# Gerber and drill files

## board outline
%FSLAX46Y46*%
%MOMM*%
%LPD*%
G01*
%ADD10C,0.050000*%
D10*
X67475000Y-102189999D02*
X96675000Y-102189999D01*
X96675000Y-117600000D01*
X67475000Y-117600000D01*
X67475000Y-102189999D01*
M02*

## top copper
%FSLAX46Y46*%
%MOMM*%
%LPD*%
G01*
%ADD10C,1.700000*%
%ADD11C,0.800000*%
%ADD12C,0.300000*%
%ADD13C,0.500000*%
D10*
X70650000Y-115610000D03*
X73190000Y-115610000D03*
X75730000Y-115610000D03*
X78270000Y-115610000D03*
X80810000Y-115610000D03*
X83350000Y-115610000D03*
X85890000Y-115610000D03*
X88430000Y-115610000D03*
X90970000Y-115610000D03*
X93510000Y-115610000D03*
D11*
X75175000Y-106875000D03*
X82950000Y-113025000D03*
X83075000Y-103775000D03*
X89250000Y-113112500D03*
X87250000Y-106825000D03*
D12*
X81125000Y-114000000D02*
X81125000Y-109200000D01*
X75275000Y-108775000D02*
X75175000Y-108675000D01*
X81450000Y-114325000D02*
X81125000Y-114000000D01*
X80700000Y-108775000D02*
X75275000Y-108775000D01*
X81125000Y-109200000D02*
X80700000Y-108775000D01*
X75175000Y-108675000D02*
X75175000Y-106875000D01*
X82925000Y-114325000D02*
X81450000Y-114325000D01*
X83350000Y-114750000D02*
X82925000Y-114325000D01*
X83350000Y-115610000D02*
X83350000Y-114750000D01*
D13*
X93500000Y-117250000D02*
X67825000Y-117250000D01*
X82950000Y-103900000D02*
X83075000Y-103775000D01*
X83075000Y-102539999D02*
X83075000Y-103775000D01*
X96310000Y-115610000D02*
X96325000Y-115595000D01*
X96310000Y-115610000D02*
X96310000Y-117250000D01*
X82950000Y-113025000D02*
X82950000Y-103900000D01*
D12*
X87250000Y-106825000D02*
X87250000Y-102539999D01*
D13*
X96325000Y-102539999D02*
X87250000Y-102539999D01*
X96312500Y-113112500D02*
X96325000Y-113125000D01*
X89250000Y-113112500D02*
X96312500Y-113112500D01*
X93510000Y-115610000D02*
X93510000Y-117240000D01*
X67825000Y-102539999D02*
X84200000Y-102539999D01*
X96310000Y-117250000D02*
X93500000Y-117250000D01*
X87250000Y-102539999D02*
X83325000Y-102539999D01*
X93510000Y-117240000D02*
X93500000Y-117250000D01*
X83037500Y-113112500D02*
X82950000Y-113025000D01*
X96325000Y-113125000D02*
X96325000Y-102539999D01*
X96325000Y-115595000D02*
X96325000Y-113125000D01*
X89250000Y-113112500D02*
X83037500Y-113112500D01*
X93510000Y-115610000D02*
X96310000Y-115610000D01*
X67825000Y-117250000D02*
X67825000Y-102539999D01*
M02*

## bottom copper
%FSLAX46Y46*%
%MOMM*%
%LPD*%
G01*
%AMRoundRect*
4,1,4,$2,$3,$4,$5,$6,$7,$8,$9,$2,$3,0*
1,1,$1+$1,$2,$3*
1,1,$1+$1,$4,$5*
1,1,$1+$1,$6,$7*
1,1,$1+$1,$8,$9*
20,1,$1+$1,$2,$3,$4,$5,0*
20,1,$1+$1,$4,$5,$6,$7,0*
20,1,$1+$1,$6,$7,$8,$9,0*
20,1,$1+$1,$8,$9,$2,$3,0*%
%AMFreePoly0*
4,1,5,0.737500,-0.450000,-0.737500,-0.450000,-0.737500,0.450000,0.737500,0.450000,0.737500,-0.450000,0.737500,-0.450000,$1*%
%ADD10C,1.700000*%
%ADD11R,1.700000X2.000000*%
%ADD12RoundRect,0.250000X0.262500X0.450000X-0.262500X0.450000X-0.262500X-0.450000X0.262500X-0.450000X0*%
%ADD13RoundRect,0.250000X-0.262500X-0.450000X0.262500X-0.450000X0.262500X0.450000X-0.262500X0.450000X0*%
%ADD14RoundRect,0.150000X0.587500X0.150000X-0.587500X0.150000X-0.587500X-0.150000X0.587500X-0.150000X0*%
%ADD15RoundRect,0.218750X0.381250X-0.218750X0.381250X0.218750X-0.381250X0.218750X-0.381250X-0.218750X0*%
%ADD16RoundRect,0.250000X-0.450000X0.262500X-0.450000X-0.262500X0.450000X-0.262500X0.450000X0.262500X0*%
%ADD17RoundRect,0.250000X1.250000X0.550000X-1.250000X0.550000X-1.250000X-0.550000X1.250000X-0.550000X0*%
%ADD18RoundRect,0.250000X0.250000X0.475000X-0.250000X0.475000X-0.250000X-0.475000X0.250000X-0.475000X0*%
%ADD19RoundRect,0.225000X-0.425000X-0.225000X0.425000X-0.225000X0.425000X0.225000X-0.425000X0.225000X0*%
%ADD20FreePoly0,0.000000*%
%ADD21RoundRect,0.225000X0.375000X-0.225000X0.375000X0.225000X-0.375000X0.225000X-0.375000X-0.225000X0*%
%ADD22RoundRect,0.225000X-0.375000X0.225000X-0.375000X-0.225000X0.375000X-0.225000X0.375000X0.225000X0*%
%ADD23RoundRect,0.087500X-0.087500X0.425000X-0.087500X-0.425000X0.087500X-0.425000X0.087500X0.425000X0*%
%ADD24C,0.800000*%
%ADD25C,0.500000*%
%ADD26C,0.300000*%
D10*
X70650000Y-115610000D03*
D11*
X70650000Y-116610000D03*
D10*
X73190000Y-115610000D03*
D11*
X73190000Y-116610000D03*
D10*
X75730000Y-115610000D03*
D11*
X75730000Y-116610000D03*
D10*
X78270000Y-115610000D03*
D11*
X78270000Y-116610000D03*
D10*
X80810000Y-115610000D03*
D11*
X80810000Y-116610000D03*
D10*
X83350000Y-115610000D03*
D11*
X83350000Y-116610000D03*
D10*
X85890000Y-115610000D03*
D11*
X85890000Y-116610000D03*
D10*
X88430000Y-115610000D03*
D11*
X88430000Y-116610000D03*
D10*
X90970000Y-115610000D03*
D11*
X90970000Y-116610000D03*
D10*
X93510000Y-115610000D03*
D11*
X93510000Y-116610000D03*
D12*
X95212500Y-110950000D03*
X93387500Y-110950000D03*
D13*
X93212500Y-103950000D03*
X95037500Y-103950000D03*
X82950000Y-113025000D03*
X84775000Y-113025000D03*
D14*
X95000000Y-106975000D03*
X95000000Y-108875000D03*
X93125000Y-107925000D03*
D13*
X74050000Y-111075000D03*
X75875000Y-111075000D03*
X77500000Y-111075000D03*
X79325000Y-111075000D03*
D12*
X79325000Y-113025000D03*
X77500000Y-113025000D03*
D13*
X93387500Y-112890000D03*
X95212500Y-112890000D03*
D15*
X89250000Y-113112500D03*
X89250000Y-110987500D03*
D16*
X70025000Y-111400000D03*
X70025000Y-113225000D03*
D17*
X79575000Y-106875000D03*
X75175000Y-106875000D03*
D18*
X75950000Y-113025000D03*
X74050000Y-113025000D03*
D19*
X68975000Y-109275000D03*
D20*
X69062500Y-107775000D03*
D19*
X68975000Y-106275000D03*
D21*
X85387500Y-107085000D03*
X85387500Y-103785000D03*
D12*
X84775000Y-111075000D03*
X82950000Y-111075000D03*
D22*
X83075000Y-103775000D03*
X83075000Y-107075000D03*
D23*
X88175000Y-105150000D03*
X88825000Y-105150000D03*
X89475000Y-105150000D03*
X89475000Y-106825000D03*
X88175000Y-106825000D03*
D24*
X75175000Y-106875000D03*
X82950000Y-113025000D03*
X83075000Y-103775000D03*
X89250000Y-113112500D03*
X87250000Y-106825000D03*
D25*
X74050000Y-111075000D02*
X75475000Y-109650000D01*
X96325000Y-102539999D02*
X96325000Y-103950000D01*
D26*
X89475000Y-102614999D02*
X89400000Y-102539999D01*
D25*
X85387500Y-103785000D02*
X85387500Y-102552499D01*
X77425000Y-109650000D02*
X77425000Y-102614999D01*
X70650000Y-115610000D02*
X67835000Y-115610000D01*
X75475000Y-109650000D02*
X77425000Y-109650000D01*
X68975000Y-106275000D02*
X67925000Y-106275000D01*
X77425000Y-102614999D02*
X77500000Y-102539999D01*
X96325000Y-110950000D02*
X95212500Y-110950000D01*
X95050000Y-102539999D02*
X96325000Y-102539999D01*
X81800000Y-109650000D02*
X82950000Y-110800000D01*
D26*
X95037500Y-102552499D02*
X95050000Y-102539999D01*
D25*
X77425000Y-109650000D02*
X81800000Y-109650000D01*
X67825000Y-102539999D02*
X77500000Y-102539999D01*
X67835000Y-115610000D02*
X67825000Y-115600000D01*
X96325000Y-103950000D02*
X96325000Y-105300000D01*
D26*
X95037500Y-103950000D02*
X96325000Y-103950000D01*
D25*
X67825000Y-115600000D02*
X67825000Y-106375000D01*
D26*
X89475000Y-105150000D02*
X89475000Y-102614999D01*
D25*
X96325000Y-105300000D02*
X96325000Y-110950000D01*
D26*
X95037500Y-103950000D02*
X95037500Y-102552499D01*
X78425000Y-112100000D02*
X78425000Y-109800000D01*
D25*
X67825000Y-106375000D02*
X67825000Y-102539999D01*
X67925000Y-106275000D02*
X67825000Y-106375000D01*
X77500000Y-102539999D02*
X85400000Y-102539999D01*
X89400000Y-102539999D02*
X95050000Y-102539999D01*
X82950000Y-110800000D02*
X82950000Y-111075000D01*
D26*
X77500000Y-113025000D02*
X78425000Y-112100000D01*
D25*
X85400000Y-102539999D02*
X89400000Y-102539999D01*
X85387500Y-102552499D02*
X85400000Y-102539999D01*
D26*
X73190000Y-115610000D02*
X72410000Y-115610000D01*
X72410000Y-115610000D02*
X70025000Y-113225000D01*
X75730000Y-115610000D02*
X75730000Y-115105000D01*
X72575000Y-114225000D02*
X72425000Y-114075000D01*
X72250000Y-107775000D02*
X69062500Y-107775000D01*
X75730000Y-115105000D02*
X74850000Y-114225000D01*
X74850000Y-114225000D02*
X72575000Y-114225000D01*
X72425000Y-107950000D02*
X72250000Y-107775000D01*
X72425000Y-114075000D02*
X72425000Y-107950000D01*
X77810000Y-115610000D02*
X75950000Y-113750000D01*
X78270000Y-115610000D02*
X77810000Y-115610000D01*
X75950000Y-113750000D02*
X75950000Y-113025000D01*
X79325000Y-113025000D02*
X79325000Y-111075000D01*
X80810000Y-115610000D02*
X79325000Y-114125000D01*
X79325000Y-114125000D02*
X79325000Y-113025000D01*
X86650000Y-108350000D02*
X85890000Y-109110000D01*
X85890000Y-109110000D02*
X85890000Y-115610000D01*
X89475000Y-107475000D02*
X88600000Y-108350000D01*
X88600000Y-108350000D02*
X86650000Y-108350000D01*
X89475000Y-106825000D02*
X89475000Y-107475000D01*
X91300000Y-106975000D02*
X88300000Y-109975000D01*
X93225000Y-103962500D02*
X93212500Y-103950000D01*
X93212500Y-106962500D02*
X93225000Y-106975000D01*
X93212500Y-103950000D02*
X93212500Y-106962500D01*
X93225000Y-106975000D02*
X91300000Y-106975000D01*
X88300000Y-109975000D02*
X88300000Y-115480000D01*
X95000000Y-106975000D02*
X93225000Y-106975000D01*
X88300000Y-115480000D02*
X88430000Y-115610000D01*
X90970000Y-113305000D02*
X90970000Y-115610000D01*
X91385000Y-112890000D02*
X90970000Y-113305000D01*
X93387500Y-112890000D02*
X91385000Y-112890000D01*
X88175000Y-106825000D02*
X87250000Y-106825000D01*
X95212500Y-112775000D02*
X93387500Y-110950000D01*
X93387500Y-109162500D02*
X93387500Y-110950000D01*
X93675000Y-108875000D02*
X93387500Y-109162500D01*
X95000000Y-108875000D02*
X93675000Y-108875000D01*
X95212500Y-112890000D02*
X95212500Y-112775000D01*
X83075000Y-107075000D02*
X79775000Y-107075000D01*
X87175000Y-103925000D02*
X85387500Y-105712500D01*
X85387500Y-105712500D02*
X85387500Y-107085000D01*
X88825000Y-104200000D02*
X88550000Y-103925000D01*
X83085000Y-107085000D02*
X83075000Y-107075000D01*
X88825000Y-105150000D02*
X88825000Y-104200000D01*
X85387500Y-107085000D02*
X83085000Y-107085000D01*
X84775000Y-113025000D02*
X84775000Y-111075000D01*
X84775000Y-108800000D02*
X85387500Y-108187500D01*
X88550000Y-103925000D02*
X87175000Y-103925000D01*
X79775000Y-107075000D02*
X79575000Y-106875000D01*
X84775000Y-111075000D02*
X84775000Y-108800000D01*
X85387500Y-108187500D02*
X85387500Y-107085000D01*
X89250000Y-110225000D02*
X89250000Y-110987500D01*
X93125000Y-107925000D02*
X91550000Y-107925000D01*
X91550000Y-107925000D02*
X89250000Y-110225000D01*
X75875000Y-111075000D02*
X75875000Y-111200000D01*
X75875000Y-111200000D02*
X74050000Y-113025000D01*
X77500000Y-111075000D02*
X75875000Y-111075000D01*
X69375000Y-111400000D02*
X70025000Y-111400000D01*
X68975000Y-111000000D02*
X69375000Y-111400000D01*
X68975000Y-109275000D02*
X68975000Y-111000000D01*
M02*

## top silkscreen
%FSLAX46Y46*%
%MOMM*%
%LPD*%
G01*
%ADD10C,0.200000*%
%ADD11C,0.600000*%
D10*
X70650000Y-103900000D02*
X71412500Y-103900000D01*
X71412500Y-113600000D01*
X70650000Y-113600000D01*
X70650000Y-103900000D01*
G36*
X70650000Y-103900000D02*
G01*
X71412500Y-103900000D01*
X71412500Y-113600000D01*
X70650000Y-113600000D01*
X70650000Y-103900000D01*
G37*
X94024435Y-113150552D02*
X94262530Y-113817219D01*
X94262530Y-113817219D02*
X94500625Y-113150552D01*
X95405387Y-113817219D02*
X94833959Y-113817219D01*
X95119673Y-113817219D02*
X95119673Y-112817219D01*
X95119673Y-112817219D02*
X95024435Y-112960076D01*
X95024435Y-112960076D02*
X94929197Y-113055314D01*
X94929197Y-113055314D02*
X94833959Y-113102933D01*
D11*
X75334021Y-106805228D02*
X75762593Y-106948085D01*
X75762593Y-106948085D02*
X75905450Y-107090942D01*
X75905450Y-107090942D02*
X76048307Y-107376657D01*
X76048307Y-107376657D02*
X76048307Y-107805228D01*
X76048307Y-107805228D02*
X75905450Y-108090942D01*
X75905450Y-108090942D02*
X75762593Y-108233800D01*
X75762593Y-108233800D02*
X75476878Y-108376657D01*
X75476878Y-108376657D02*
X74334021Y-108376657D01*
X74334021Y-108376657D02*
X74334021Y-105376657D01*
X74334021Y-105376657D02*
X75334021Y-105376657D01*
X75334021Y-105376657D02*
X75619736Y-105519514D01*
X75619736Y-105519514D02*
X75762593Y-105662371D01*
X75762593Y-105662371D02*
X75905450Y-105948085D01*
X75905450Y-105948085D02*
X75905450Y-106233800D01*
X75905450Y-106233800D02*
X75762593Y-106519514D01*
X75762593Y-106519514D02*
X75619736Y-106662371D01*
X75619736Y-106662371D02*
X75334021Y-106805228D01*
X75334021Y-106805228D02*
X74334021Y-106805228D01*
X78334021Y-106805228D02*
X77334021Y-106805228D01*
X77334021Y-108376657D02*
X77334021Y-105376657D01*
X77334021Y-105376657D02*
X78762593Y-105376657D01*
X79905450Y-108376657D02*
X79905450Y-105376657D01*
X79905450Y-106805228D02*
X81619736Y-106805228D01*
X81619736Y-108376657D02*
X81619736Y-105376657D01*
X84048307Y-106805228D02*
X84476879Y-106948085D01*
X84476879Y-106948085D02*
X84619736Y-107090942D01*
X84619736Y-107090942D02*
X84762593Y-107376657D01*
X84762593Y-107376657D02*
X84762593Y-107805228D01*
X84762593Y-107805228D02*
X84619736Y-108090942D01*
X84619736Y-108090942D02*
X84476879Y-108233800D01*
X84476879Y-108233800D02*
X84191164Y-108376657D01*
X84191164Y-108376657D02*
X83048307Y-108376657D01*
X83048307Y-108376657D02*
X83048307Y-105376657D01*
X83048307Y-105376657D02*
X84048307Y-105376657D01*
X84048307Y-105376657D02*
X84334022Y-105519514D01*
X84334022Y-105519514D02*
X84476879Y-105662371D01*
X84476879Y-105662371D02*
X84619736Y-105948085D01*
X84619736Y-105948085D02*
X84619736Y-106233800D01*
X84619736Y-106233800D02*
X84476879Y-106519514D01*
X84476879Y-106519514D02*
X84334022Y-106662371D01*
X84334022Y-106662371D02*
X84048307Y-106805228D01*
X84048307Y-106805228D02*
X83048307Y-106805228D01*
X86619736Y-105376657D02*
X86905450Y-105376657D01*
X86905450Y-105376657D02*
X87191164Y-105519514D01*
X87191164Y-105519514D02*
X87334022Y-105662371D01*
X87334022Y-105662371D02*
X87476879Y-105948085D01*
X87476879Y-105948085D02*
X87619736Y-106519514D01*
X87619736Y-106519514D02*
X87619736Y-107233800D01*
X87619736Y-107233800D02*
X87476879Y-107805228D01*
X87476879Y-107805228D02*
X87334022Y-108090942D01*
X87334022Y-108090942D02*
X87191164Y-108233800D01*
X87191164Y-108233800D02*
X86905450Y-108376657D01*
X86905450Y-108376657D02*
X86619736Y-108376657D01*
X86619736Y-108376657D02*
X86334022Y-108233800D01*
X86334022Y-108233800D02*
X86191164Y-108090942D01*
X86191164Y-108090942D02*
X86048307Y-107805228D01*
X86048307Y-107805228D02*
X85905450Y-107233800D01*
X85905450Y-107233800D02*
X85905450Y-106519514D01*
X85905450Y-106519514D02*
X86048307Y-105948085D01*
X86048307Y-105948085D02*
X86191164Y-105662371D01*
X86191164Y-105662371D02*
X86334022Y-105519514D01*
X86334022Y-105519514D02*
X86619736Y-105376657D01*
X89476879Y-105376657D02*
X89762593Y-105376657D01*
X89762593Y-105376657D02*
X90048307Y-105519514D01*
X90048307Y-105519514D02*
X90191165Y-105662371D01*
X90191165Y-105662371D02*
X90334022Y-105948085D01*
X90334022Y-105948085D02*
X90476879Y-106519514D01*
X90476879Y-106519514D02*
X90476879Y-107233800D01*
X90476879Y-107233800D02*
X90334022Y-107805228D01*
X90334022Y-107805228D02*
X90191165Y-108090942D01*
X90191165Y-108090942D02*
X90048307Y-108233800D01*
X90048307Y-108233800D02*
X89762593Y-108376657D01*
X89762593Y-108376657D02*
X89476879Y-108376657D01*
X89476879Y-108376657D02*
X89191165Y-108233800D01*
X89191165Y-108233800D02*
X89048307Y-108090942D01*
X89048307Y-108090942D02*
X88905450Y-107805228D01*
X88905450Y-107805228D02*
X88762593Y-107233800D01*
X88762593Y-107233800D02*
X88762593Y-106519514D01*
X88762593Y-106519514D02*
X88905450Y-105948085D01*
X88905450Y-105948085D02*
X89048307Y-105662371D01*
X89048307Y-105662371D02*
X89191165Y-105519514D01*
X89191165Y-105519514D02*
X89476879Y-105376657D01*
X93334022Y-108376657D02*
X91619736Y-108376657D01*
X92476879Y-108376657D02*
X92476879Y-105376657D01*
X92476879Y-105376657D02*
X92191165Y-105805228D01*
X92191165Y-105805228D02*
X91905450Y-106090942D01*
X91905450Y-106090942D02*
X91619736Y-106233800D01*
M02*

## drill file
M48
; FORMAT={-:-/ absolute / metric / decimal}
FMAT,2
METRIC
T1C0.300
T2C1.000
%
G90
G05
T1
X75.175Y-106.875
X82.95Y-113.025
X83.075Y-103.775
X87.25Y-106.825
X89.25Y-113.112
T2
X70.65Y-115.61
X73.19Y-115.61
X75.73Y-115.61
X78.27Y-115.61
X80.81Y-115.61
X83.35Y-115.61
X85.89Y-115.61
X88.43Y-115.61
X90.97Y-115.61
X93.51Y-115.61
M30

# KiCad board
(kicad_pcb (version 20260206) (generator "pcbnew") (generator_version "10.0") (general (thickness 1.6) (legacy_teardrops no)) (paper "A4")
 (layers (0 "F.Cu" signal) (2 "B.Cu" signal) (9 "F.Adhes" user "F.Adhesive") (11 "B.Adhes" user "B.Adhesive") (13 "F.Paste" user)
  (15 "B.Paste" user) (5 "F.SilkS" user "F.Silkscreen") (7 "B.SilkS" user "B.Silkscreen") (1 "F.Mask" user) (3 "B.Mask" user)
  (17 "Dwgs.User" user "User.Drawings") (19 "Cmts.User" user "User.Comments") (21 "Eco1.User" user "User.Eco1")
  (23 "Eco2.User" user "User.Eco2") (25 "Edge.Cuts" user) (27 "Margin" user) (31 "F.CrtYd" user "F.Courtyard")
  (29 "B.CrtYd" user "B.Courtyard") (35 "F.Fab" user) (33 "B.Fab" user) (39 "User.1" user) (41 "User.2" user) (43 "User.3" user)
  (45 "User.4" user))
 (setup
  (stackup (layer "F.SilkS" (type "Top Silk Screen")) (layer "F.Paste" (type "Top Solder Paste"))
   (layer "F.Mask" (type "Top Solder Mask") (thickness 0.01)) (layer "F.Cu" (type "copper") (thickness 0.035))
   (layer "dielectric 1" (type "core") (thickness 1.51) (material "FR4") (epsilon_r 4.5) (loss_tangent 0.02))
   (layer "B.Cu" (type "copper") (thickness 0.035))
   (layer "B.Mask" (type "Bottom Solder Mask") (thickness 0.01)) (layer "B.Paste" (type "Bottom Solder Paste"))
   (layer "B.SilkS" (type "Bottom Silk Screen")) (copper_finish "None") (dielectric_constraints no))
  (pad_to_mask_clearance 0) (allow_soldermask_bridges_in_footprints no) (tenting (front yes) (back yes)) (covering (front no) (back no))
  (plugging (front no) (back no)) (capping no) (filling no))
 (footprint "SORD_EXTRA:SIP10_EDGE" (layer "F.Cu") (at 70.65 115.61)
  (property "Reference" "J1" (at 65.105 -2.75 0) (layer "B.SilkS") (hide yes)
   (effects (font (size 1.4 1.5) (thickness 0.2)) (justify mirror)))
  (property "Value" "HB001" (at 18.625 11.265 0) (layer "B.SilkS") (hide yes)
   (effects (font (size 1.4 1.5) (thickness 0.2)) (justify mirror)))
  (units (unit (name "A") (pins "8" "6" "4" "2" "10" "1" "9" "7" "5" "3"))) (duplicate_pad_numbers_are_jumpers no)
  (pad "1" thru_hole circle (at 0 0) (size 1.7 1.7) (drill 1) (layers "*.Cu" "*.Mask") (remove_unused_layers no) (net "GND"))
  (pad "1" smd rect (at 0 1 180) (size 1.7 2) (layers "B.Cu" "B.Mask") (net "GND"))
  (pad "2" thru_hole circle (at 2.54 0) (size 1.7 1.7) (drill 1) (layers "*.Cu" "*.Mask") (remove_unused_layers no) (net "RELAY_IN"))
  (pad "2" smd rect (at 2.54 1 180) (size 1.7 2) (layers "B.Cu" "B.Mask") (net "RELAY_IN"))
  (pad "3" thru_hole circle (at 5.08 0) (size 1.7 1.7) (drill 1) (layers "*.Cu" "*.Mask") (remove_unused_layers no) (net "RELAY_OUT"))
  (pad "3" smd rect (at 5.08 1 180) (size 1.7 2) (layers "B.Cu" "B.Mask") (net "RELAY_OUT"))
  (pad "4" thru_hole circle (at 7.62 0) (size 1.7 1.7) (drill 1) (layers "*.Cu" "*.Mask") (remove_unused_layers no) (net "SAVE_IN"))
  (pad "4" smd rect (at 7.62 1 180) (size 1.7 2) (layers "B.Cu" "B.Mask") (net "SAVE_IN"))
  (pad "5" thru_hole circle (at 10.16 0) (size 1.7 1.7) (drill 1) (layers "*.Cu" "*.Mask") (remove_unused_layers no) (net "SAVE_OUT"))
  (pad "5" smd rect (at 10.16 1 180) (size 1.7 2) (layers "B.Cu" "B.Mask") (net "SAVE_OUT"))
  (pad "6" thru_hole circle (at 12.7 0) (size 1.7 1.7) (drill 1) (layers "*.Cu" "*.Mask") (remove_unused_layers no) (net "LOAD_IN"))
  (pad "6" smd rect (at 12.7 1 180) (size 1.7 2) (layers "B.Cu" "B.Mask") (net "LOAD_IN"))
  (pad "7" thru_hole circle (at 15.24 0) (size 1.7 1.7) (drill 1) (layers "*.Cu" "*.Mask") (remove_unused_layers no) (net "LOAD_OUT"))
  (pad "7" smd rect (at 15.24 1 180) (size 1.7 2) (layers "B.Cu" "B.Mask") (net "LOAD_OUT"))
  (pad "8" thru_hole circle (at 17.78 0) (size 1.7 1.7) (drill 1) (layers "*.Cu" "*.Mask") (remove_unused_layers no) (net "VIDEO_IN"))
  (pad "8" smd rect (at 17.78 1 180) (size 1.7 2) (layers "B.Cu" "B.Mask") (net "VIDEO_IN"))
  (pad "9" thru_hole circle (at 20.32 0) (size 1.7 1.7) (drill 1) (layers "*.Cu" "*.Mask") (remove_unused_layers no) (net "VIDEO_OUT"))
  (pad "9" smd rect (at 20.32 1 180) (size 1.7 2) (layers "B.Cu" "B.Mask") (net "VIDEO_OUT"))
  (pad "10" thru_hole circle (at 22.86 0) (size 1.7 1.7) (drill 1) (layers "*.Cu" "*.Mask") (remove_unused_layers no) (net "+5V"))
  (pad "10" smd rect (at 22.86 1 180) (size 1.7 2) (layers "B.Cu" "B.Mask") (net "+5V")))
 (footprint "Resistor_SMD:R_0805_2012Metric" (layer "B.Cu") (at 94.3 110.95 180)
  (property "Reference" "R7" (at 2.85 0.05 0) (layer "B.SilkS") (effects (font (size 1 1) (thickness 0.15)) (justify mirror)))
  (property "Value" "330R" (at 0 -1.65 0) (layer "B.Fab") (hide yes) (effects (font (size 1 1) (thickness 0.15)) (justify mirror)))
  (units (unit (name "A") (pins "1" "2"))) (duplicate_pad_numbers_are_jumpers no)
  (pad "1" smd roundrect (at -0.9125 0 180) (size 1.025 1.4) (layers "B.Cu" "B.Mask" "B.Paste") (roundrect_rratio 0.243902) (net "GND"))
  (pad "2" smd roundrect (at 0.9125 0 180) (size 1.025 1.4) (layers "B.Cu" "B.Mask" "B.Paste") (roundrect_rratio 0.243902)
   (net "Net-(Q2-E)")))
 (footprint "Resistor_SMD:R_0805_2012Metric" (layer "B.Cu") (at 94.125 103.95)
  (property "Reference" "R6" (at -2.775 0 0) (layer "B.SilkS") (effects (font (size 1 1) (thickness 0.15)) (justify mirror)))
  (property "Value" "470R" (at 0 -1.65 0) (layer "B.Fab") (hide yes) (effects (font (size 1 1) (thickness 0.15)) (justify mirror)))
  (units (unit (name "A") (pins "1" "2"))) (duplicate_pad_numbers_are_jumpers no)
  (pad "1" smd roundrect (at -0.9125 0) (size 1.025 1.4) (layers "B.Cu" "B.Mask" "B.Paste") (roundrect_rratio 0.243902) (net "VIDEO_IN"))
  (pad "2" smd roundrect (at 0.9125 0) (size 1.025 1.4) (layers "B.Cu" "B.Mask" "B.Paste") (roundrect_rratio 0.243902) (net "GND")))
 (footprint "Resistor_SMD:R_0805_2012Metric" (layer "B.Cu") (at 83.8625 113.025)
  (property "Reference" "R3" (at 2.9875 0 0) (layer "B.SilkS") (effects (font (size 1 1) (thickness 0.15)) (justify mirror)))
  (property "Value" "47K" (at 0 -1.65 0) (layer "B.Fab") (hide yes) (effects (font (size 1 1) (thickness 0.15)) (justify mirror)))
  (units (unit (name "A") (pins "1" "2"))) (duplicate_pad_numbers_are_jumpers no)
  (pad "1" smd roundrect (at -0.9125 0) (size 1.025 1.4) (layers "B.Cu" "B.Mask" "B.Paste") (roundrect_rratio 0.243902) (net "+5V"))
  (pad "2" smd roundrect (at 0.9125 0) (size 1.025 1.4) (layers "B.Cu" "B.Mask" "B.Paste") (roundrect_rratio 0.243902) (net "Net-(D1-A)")))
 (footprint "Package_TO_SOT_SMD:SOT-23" (layer "B.Cu") (at 94.0625 107.925 180)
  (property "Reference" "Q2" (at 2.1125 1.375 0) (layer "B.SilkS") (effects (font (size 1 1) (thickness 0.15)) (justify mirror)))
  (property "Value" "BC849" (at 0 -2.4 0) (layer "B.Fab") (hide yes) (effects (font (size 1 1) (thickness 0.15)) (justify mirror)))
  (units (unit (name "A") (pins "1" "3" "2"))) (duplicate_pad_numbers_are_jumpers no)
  (pad "1" smd roundrect (at -0.9375 0.95 180) (size 1.475 0.6) (layers "B.Cu" "B.Mask" "B.Paste") (roundrect_rratio 0.25) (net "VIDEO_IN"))
  (pad "2" smd roundrect (at -0.9375 -0.95 180) (size 1.475 0.6) (layers "B.Cu" "B.Mask" "B.Paste") (roundrect_rratio 0.25)
   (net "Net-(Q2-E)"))
  (pad "3" smd roundrect (at 0.9375 0 180) (size 1.475 0.6) (layers "B.Cu" "B.Mask" "B.Paste") (roundrect_rratio 0.25) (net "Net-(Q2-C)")))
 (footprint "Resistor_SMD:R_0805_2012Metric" (layer "B.Cu") (at 74.9625 111.075)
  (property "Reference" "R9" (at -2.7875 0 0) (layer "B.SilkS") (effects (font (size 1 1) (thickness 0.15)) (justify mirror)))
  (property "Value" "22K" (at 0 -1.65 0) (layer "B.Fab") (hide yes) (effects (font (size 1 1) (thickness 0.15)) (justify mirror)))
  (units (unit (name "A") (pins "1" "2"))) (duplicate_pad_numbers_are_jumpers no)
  (pad "1" smd roundrect (at -0.9125 0) (size 1.025 1.4) (layers "B.Cu" "B.Mask" "B.Paste") (roundrect_rratio 0.243902) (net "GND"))
  (pad "2" smd roundrect (at 0.9125 0) (size 1.025 1.4) (layers "B.Cu" "B.Mask" "B.Paste") (roundrect_rratio 0.243902) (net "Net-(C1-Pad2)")))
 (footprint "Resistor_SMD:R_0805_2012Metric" (layer "B.Cu") (at 78.4125 111.075)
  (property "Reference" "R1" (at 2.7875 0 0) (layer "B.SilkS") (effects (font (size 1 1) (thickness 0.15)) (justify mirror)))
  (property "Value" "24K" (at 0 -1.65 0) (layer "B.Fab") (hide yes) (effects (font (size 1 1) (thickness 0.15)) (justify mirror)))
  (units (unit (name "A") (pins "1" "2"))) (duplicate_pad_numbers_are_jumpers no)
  (pad "1" smd roundrect (at -0.9125 0) (size 1.025 1.4) (layers "B.Cu" "B.Mask" "B.Paste") (roundrect_rratio 0.243902)
   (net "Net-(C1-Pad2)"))
  (pad "2" smd roundrect (at 0.9125 0) (size 1.025 1.4) (layers "B.Cu" "B.Mask" "B.Paste") (roundrect_rratio 0.243902) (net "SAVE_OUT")))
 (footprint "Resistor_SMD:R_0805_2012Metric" (layer "B.Cu") (at 78.4125 113.025 180)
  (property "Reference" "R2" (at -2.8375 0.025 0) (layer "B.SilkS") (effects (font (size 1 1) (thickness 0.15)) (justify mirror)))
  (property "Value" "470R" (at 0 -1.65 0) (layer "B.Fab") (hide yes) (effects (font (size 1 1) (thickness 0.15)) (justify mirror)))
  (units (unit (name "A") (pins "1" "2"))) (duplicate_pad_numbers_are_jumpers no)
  (pad "1" smd roundrect (at -0.9125 0 180) (size 1.025 1.4) (layers "B.Cu" "B.Mask" "B.Paste") (roundrect_rratio 0.243902) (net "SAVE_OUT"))
  (pad "2" smd roundrect (at 0.9125 0 180) (size 1.025 1.4) (layers "B.Cu" "B.Mask" "B.Paste") (roundrect_rratio 0.243902) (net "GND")))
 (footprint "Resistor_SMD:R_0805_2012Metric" (layer "B.Cu") (at 94.3 112.89)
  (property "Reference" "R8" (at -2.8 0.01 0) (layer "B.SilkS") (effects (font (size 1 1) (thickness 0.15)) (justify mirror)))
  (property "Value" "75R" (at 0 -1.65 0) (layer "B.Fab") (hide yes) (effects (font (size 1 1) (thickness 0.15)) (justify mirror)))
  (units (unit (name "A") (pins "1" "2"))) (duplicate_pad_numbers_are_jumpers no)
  (pad "1" smd roundrect (at -0.9125 0) (size 1.025 1.4) (layers "B.Cu" "B.Mask" "B.Paste") (roundrect_rratio 0.243902) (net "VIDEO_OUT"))
  (pad "2" smd roundrect (at 0.9125 0) (size 1.025 1.4) (layers "B.Cu" "B.Mask" "B.Paste") (roundrect_rratio 0.243902) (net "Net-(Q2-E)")))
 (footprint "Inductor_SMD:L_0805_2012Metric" (layer "B.Cu") (at 89.25 112.05 90)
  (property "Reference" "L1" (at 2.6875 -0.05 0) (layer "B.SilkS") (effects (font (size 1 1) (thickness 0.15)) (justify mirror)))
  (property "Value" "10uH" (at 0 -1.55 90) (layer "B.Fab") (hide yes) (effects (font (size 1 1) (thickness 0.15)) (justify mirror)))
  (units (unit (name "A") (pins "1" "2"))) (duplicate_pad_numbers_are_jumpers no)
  (pad "1" smd roundrect (at -1.0625 0 90) (size 0.875 1.2) (layers "B.Cu" "B.Mask" "B.Paste") (roundrect_rratio 0.25) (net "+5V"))
  (pad "2" smd roundrect (at 1.0625 0 90) (size 0.875 1.2) (layers "B.Cu" "B.Mask" "B.Paste") (roundrect_rratio 0.25) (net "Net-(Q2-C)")))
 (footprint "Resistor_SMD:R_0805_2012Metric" (layer "B.Cu") (at 70.025 112.3125 -90)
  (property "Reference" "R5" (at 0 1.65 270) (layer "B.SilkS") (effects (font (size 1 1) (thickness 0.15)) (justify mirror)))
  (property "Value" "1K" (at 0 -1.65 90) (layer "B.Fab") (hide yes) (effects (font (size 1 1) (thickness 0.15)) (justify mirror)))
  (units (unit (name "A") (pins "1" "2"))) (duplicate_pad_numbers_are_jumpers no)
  (pad "1" smd roundrect (at -0.9125 0 270) (size 1.025 1.4) (layers "B.Cu" "B.Mask" "B.Paste") (roundrect_rratio 0.243902)
   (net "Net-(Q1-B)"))
  (pad "2" smd roundrect (at 0.9125 0 270) (size 1.025 1.4) (layers "B.Cu" "B.Mask" "B.Paste") (roundrect_rratio 0.243902) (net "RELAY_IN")))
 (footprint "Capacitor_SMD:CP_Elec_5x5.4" (layer "B.Cu") (at 77.375 106.875 180)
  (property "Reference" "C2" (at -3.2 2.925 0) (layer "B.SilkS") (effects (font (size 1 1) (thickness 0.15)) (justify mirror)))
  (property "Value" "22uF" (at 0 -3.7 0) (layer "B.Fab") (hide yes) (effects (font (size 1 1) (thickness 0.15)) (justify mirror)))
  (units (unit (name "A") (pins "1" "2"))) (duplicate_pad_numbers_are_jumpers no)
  (pad "1" smd roundrect (at -2.2 0 180) (size 3 1.6) (layers "B.Cu" "B.Mask" "B.Paste") (roundrect_rratio 0.15625) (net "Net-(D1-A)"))
  (pad "2" smd roundrect (at 2.2 0 180) (size 3 1.6) (layers "B.Cu" "B.Mask" "B.Paste") (roundrect_rratio 0.15625) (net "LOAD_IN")))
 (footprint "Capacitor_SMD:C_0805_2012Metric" (layer "B.Cu") (at 75 113.025 180)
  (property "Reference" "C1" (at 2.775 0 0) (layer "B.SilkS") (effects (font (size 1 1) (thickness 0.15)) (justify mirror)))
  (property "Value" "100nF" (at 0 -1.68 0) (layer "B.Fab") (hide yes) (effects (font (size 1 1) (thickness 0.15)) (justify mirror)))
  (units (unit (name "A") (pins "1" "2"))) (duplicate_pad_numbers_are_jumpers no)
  (pad "1" smd roundrect (at -0.95 0 180) (size 1 1.45) (layers "B.Cu" "B.Mask" "B.Paste") (roundrect_rratio 0.25) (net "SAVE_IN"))
  (pad "2" smd roundrect (at 0.95 0 180) (size 1 1.45) (layers "B.Cu" "B.Mask" "B.Paste") (roundrect_rratio 0.25) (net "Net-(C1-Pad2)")))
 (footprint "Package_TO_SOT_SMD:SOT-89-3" (layer "B.Cu") (at 70.925 107.775)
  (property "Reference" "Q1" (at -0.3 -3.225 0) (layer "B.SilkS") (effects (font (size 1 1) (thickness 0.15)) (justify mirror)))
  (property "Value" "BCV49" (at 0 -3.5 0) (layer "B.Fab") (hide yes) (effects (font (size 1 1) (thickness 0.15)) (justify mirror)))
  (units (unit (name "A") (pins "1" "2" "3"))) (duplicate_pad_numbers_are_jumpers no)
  (pad "1" smd roundrect (at -1.95 1.5) (size 1.3 0.9) (layers "B.Cu" "B.Mask" "B.Paste") (roundrect_rratio 0.25) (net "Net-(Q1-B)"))
  (pad "2" smd custom (at -1.8625 0) (size 1.475 0.9) (layers "B.Cu" "B.Mask" "B.Paste") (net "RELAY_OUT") (zone_connect 2)
   (thermal_bridge_angle 45) (options (clearance outline) (anchor rect)) (primitives))
  (pad "3" smd roundrect (at -1.95 -1.5) (size 1.3 0.9) (layers "B.Cu" "B.Mask" "B.Paste") (roundrect_rratio 0.25) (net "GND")))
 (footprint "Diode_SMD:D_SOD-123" (layer "B.Cu") (at 85.3875 105.435 90)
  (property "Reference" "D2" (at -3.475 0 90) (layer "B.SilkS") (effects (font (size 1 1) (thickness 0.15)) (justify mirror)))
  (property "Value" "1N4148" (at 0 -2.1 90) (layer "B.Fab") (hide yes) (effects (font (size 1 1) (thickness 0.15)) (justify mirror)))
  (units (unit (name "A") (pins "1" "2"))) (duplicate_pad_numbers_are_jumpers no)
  (pad "1" smd roundrect (at -1.65 0 90) (size 0.9 1.2) (layers "B.Cu" "B.Mask" "B.Paste") (roundrect_rratio 0.25) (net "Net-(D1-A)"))
  (pad "2" smd roundrect (at 1.65 0 90) (size 0.9 1.2) (layers "B.Cu" "B.Mask" "B.Paste") (roundrect_rratio 0.25) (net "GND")))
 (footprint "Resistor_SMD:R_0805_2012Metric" (layer "B.Cu") (at 83.8625 111.075 180)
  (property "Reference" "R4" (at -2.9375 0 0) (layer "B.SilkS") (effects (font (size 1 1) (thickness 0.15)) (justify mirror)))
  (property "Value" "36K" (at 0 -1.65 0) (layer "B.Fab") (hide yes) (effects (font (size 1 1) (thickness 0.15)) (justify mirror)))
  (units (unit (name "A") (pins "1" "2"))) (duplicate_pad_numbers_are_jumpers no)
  (pad "1" smd roundrect (at -0.9125 0 180) (size 1.025 1.4) (layers "B.Cu" "B.Mask" "B.Paste") (roundrect_rratio 0.243902)
   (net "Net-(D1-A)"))
  (pad "2" smd roundrect (at 0.9125 0 180) (size 1.025 1.4) (layers "B.Cu" "B.Mask" "B.Paste") (roundrect_rratio 0.243902) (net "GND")))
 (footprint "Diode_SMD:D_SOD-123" (layer "B.Cu") (at 83.075 105.425 -90)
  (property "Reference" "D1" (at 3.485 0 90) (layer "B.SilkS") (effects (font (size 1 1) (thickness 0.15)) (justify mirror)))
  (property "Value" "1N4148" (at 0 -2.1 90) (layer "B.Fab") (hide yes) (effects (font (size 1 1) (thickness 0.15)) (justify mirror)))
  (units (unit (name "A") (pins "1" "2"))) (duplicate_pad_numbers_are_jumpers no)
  (pad "1" smd roundrect (at -1.65 0 270) (size 0.9 1.2) (layers "B.Cu" "B.Mask" "B.Paste") (roundrect_rratio 0.25) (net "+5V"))
  (pad "2" smd roundrect (at 1.65 0 270) (size 0.9 1.2) (layers "B.Cu" "B.Mask" "B.Paste") (roundrect_rratio 0.25) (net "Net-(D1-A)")))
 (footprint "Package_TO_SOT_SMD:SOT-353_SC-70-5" (layer "B.Cu") (at 88.825 105.9875 -90)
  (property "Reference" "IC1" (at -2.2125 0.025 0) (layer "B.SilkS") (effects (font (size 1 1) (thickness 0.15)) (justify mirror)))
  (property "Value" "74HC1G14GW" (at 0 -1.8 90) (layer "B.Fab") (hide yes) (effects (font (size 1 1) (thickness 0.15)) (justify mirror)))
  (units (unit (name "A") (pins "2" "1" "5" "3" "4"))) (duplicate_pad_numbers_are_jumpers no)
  (pad "1" smd roundrect (at -0.8375 0.65 270) (size 1.025 0.35) (layers "B.Cu" "B.Mask" "B.Paste") (roundrect_rratio 0.25)
   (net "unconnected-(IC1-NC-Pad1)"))
  (pad "2" smd roundrect (at -0.8375 0 270) (size 1.025 0.35) (layers "B.Cu" "B.Mask" "B.Paste") (roundrect_rratio 0.25) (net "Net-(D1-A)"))
  (pad "3" smd roundrect (at -0.8375 -0.65 270) (size 1.025 0.35) (layers "B.Cu" "B.Mask" "B.Paste") (roundrect_rratio 0.25) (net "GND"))
  (pad "4" smd roundrect (at 0.8375 -0.65 270) (size 1.025 0.35) (layers "B.Cu" "B.Mask" "B.Paste") (roundrect_rratio 0.25) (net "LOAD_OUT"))
  (pad "5" smd roundrect (at 0.8375 0.65 270) (size 1.025 0.35) (layers "B.Cu" "B.Mask" "B.Paste") (roundrect_rratio 0.25) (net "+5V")))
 (gr_rect (start 70.65 103.9) (end 71.4125 113.6) (stroke (width 0.2) (type solid)) (fill yes) (layer "F.SilkS"))
 (gr_rect (start 67.475 102.189999) (end 96.675 117.6) (stroke (width 0.05) (type default)) (fill no) (layer "Edge.Cuts"))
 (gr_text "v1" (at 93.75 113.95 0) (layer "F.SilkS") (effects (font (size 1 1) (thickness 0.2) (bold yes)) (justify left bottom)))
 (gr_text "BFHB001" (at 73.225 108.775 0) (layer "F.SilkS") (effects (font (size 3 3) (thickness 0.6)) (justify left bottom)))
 (segment (start 74.05 111.075) (end 75.475 109.65) (width 0.5) (layer "B.Cu") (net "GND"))
 (segment (start 96.325 102.539999) (end 96.325 103.95) (width 0.5) (layer "B.Cu") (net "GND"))
 (segment (start 89.475 102.614999) (end 89.4 102.539999) (width 0.3) (layer "B.Cu") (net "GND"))
 (segment (start 85.3875 103.785) (end 85.3875 102.552499) (width 0.5) (layer "B.Cu") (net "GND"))
 (segment (start 77.425 109.65) (end 77.425 102.614999) (width 0.5) (layer "B.Cu") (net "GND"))
 (segment (start 70.65 115.61) (end 67.835 115.61) (width 0.5) (layer "B.Cu") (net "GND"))
 (segment (start 75.475 109.65) (end 77.425 109.65) (width 0.5) (layer "B.Cu") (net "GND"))
 (segment (start 68.975 106.275) (end 67.925 106.275) (width 0.5) (layer "B.Cu") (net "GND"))
 (segment (start 77.425 102.614999) (end 77.5 102.539999) (width 0.5) (layer "B.Cu") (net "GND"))
 (segment (start 96.325 110.95) (end 95.2125 110.95) (width 0.5) (layer "B.Cu") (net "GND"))
 (segment (start 95.05 102.539999) (end 96.325 102.539999) (width 0.5) (layer "B.Cu") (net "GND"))
 (segment (start 81.8 109.65) (end 82.95 110.8) (width 0.5) (layer "B.Cu") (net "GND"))
 (segment (start 95.0375 102.552499) (end 95.05 102.539999) (width 0.3) (layer "B.Cu") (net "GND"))
 (segment (start 77.425 109.65) (end 81.8 109.65) (width 0.5) (layer "B.Cu") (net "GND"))
 (segment (start 67.825 102.539999) (end 77.5 102.539999) (width 0.5) (layer "B.Cu") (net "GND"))
 (segment (start 67.835 115.61) (end 67.825 115.6) (width 0.5) (layer "B.Cu") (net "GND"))
 (segment (start 96.325 103.95) (end 96.325 105.3) (width 0.5) (layer "B.Cu") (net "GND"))
 (segment (start 95.0375 103.95) (end 96.325 103.95) (width 0.3) (layer "B.Cu") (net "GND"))
 (segment (start 67.825 115.6) (end 67.825 106.375) (width 0.5) (layer "B.Cu") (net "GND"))
 (segment (start 89.475 105.15) (end 89.475 102.614999) (width 0.3) (layer "B.Cu") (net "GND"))
 (segment (start 96.325 105.3) (end 96.325 110.95) (width 0.5) (layer "B.Cu") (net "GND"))
 (segment (start 95.0375 103.95) (end 95.0375 102.552499) (width 0.3) (layer "B.Cu") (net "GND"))
 (segment (start 78.425 112.1) (end 78.425 109.8) (width 0.3) (layer "B.Cu") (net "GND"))
 (segment (start 67.825 106.375) (end 67.825 102.539999) (width 0.5) (layer "B.Cu") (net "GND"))
 (segment (start 67.925 106.275) (end 67.825 106.375) (width 0.5) (layer "B.Cu") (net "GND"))
 (segment (start 77.5 102.539999) (end 85.4 102.539999) (width 0.5) (layer "B.Cu") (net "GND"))
 (segment (start 89.4 102.539999) (end 95.05 102.539999) (width 0.5) (layer "B.Cu") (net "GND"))
 (segment (start 82.95 110.8) (end 82.95 111.075) (width 0.5) (layer "B.Cu") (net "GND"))
 (segment (start 77.5 113.025) (end 78.425 112.1) (width 0.3) (layer "B.Cu") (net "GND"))
 (segment (start 85.4 102.539999) (end 89.4 102.539999) (width 0.5) (layer "B.Cu") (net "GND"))
 (segment (start 85.3875 102.552499) (end 85.4 102.539999) (width 0.5) (layer "B.Cu") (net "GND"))
 (segment (start 73.19 115.61) (end 72.41 115.61) (width 0.3) (layer "B.Cu") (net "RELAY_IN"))
 (segment (start 72.41 115.61) (end 70.025 113.225) (width 0.3) (layer "B.Cu") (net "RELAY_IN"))
 (segment (start 75.73 115.61) (end 75.73 115.105) (width 0.3) (layer "B.Cu") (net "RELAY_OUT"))
 (segment (start 72.575 114.225) (end 72.425 114.075) (width 0.3) (layer "B.Cu") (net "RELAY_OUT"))
 (segment (start 72.25 107.775) (end 69.0625 107.775) (width 0.3) (layer "B.Cu") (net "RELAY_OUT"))
 (segment (start 75.73 115.105) (end 74.85 114.225) (width 0.3) (layer "B.Cu") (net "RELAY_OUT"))
 (segment (start 74.85 114.225) (end 72.575 114.225) (width 0.3) (layer "B.Cu") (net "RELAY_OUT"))
 (segment (start 72.425 107.95) (end 72.25 107.775) (width 0.3) (layer "B.Cu") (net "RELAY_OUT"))
 (segment (start 72.425 114.075) (end 72.425 107.95) (width 0.3) (layer "B.Cu") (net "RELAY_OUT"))
 (segment (start 77.81 115.61) (end 75.95 113.75) (width 0.3) (layer "B.Cu") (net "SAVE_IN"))
 (segment (start 78.27 115.61) (end 77.81 115.61) (width 0.3) (layer "B.Cu") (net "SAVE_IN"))
 (segment (start 75.95 113.75) (end 75.95 113.025) (width 0.3) (layer "B.Cu") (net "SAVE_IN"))
 (segment (start 79.325 113.025) (end 79.325 111.075) (width 0.3) (layer "B.Cu") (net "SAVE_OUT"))
 (segment (start 80.81 115.61) (end 79.325 114.125) (width 0.3) (layer "B.Cu") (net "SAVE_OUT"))
 (segment (start 79.325 114.125) (end 79.325 113.025) (width 0.3) (layer "B.Cu") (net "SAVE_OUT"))
 (segment (start 81.125 114) (end 81.125 109.2) (width 0.3) (layer "F.Cu") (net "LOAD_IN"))
 (segment (start 75.275 108.775) (end 75.175 108.675) (width 0.3) (layer "F.Cu") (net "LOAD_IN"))
 (segment (start 81.45 114.325) (end 81.125 114) (width 0.3) (layer "F.Cu") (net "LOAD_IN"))
 (segment (start 80.7 108.775) (end 75.275 108.775) (width 0.3) (layer "F.Cu") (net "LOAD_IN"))
 (segment (start 81.125 109.2) (end 80.7 108.775) (width 0.3) (layer "F.Cu") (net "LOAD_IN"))
 (segment (start 75.175 108.675) (end 75.175 106.875) (width 0.3) (layer "F.Cu") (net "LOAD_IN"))
 (segment (start 82.925 114.325) (end 81.45 114.325) (width 0.3) (layer "F.Cu") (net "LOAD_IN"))
 (segment (start 83.35 114.75) (end 82.925 114.325) (width 0.3) (layer "F.Cu") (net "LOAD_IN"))
 (segment (start 83.35 115.61) (end 83.35 114.75) (width 0.3) (layer "F.Cu") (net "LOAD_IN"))
 (via (at 75.175 106.875) (size 0.8) (drill 0.3) (layers "F.Cu" "B.Cu") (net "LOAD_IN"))
 (segment (start 86.65 108.35) (end 85.89 109.11) (width 0.3) (layer "B.Cu") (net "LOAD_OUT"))
 (segment (start 85.89 109.11) (end 85.89 115.61) (width 0.3) (layer "B.Cu") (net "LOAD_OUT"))
 (segment (start 89.475 107.475) (end 88.6 108.35) (width 0.3) (layer "B.Cu") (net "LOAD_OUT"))
 (segment (start 88.6 108.35) (end 86.65 108.35) (width 0.3) (layer "B.Cu") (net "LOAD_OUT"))
 (segment (start 89.475 106.825) (end 89.475 107.475) (width 0.3) (layer "B.Cu") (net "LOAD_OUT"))
 (segment (start 91.3 106.975) (end 88.3 109.975) (width 0.3) (layer "B.Cu") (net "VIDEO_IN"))
 (segment (start 93.225 103.9625) (end 93.2125 103.95) (width 0.3) (layer "B.Cu") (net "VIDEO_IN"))
 (segment (start 93.2125 106.9625) (end 93.225 106.975) (width 0.3) (layer "B.Cu") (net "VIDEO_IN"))
 (segment (start 93.2125 103.95) (end 93.2125 106.9625) (width 0.3) (layer "B.Cu") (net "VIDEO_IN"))
 (segment (start 93.225 106.975) (end 91.3 106.975) (width 0.3) (layer "B.Cu") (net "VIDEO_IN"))
 (segment (start 88.3 109.975) (end 88.3 115.48) (width 0.3) (layer "B.Cu") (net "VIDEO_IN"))
 (segment (start 95 106.975) (end 93.225 106.975) (width 0.3) (layer "B.Cu") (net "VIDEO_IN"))
 (segment (start 88.3 115.48) (end 88.43 115.61) (width 0.3) (layer "B.Cu") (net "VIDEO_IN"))
 (segment (start 90.97 113.305) (end 90.97 115.61) (width 0.3) (layer "B.Cu") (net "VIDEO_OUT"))
 (segment (start 91.385 112.89) (end 90.97 113.305) (width 0.3) (layer "B.Cu") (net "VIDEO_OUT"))
 (segment (start 93.3875 112.89) (end 91.385 112.89) (width 0.3) (layer "B.Cu") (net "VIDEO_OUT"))
 (segment (start 93.5 117.25) (end 67.825 117.25) (width 0.5) (layer "F.Cu") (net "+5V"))
 (segment (start 82.95 103.9) (end 83.075 103.775) (width 0.5) (layer "F.Cu") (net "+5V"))
 (segment (start 83.075 102.539999) (end 83.075 103.775) (width 0.5) (layer "F.Cu") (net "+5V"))
 (segment (start 96.31 115.61) (end 96.325 115.595) (width 0.5) (layer "F.Cu") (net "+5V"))
 (segment (start 96.31 115.61) (end 96.31 117.25) (width 0.5) (layer "F.Cu") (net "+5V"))
 (segment (start 82.95 113.025) (end 82.95 103.9) (width 0.5) (layer "F.Cu") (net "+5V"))
 (segment (start 87.25 106.825) (end 87.25 102.539999) (width 0.3) (layer "F.Cu") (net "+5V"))
 (segment (start 96.325 102.539999) (end 87.25 102.539999) (width 0.5) (layer "F.Cu") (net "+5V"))
 (segment (start 96.3125 113.1125) (end 96.325 113.125) (width 0.5) (layer "F.Cu") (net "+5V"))
 (segment (start 89.25 113.1125) (end 96.3125 113.1125) (width 0.5) (layer "F.Cu") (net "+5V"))
 (segment (start 93.51 115.61) (end 93.51 117.24) (width 0.5) (layer "F.Cu") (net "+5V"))
 (segment (start 67.825 102.539999) (end 84.2 102.539999) (width 0.5) (layer "F.Cu") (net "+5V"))
 (segment (start 96.31 117.25) (end 93.5 117.25) (width 0.5) (layer "F.Cu") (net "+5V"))
 (segment (start 87.25 102.539999) (end 83.325 102.539999) (width 0.5) (layer "F.Cu") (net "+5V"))
 (segment (start 93.51 117.24) (end 93.5 117.25) (width 0.5) (layer "F.Cu") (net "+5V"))
 (segment (start 83.0375 113.1125) (end 82.95 113.025) (width 0.5) (layer "F.Cu") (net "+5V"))
 (segment (start 96.325 113.125) (end 96.325 102.539999) (width 0.5) (layer "F.Cu") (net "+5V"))
 (segment (start 96.325 115.595) (end 96.325 113.125) (width 0.5) (layer "F.Cu") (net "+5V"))
 (segment (start 89.25 113.1125) (end 83.0375 113.1125) (width 0.5) (layer "F.Cu") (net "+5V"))
 (segment (start 93.51 115.61) (end 96.31 115.61) (width 0.5) (layer "F.Cu") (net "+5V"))
 (segment (start 67.825 117.25) (end 67.825 102.539999) (width 0.5) (layer "F.Cu") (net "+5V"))
 (via (at 82.95 113.025) (size 0.8) (drill 0.3) (layers "F.Cu" "B.Cu") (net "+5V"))
 (via (at 83.075 103.775) (size 0.8) (drill 0.3) (layers "F.Cu" "B.Cu") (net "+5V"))
 (via (at 89.25 113.1125) (size 0.8) (drill 0.3) (layers "F.Cu" "B.Cu") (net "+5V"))
 (via (at 87.25 106.825) (size 0.8) (drill 0.3) (layers "F.Cu" "B.Cu") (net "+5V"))
 (segment (start 88.175 106.825) (end 87.25 106.825) (width 0.3) (layer "B.Cu") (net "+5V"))
 (segment (start 95.2125 112.775) (end 93.3875 110.95) (width 0.3) (layer "B.Cu") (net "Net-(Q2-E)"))
 (segment (start 93.3875 109.1625) (end 93.3875 110.95) (width 0.3) (layer "B.Cu") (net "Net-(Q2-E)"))
 (segment (start 93.675 108.875) (end 93.3875 109.1625) (width 0.3) (layer "B.Cu") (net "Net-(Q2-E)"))
 (segment (start 95 108.875) (end 93.675 108.875) (width 0.3) (layer "B.Cu") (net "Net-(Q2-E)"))
 (segment (start 95.2125 112.89) (end 95.2125 112.775) (width 0.3) (layer "B.Cu") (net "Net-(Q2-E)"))
 (segment (start 83.075 107.075) (end 79.775 107.075) (width 0.3) (layer "B.Cu") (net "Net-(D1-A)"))
 (segment (start 87.175 103.925) (end 85.3875 105.7125) (width 0.3) (layer "B.Cu") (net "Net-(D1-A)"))
 (segment (start 85.3875 105.7125) (end 85.3875 107.085) (width 0.3) (layer "B.Cu") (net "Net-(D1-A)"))
 (segment (start 88.825 104.2) (end 88.55 103.925) (width 0.3) (layer "B.Cu") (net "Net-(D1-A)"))
 (segment (start 83.085 107.085) (end 83.075 107.075) (width 0.3) (layer "B.Cu") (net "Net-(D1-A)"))
 (segment (start 88.825 105.15) (end 88.825 104.2) (width 0.3) (layer "B.Cu") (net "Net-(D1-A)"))
 (segment (start 85.3875 107.085) (end 83.085 107.085) (width 0.3) (layer "B.Cu") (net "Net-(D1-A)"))
 (segment (start 84.775 113.025) (end 84.775 111.075) (width 0.3) (layer "B.Cu") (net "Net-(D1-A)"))
 (segment (start 84.775 108.8) (end 85.3875 108.1875) (width 0.3) (layer "B.Cu") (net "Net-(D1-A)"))
 (segment (start 88.55 103.925) (end 87.175 103.925) (width 0.3) (layer "B.Cu") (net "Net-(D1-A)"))
 (segment (start 79.775 107.075) (end 79.575 106.875) (width 0.3) (layer "B.Cu") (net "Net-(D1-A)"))
 (segment (start 84.775 111.075) (end 84.775 108.8) (width 0.3) (layer "B.Cu") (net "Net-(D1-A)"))
 (segment (start 85.3875 108.1875) (end 85.3875 107.085) (width 0.3) (layer "B.Cu") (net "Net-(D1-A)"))
 (segment (start 89.25 110.225) (end 89.25 110.9875) (width 0.3) (layer "B.Cu") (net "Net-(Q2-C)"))
 (segment (start 93.125 107.925) (end 91.55 107.925) (width 0.3) (layer "B.Cu") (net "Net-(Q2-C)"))
 (segment (start 91.55 107.925) (end 89.25 110.225) (width 0.3) (layer "B.Cu") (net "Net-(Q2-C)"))
 (segment (start 75.875 111.075) (end 75.875 111.2) (width 0.3) (layer "B.Cu") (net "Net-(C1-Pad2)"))
 (segment (start 75.875 111.2) (end 74.05 113.025) (width 0.3) (layer "B.Cu") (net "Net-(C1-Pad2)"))
 (segment (start 77.5 111.075) (end 75.875 111.075) (width 0.3) (layer "B.Cu") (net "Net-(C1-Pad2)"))
 (segment (start 69.375 111.4) (end 70.025 111.4) (width 0.3) (layer "B.Cu") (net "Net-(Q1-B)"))
 (segment (start 68.975 111) (end 69.375 111.4) (width 0.3) (layer "B.Cu") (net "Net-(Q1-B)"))
 (segment (start 68.975 109.275) (end 68.975 111) (width 0.3) (layer "B.Cu") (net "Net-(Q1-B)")))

